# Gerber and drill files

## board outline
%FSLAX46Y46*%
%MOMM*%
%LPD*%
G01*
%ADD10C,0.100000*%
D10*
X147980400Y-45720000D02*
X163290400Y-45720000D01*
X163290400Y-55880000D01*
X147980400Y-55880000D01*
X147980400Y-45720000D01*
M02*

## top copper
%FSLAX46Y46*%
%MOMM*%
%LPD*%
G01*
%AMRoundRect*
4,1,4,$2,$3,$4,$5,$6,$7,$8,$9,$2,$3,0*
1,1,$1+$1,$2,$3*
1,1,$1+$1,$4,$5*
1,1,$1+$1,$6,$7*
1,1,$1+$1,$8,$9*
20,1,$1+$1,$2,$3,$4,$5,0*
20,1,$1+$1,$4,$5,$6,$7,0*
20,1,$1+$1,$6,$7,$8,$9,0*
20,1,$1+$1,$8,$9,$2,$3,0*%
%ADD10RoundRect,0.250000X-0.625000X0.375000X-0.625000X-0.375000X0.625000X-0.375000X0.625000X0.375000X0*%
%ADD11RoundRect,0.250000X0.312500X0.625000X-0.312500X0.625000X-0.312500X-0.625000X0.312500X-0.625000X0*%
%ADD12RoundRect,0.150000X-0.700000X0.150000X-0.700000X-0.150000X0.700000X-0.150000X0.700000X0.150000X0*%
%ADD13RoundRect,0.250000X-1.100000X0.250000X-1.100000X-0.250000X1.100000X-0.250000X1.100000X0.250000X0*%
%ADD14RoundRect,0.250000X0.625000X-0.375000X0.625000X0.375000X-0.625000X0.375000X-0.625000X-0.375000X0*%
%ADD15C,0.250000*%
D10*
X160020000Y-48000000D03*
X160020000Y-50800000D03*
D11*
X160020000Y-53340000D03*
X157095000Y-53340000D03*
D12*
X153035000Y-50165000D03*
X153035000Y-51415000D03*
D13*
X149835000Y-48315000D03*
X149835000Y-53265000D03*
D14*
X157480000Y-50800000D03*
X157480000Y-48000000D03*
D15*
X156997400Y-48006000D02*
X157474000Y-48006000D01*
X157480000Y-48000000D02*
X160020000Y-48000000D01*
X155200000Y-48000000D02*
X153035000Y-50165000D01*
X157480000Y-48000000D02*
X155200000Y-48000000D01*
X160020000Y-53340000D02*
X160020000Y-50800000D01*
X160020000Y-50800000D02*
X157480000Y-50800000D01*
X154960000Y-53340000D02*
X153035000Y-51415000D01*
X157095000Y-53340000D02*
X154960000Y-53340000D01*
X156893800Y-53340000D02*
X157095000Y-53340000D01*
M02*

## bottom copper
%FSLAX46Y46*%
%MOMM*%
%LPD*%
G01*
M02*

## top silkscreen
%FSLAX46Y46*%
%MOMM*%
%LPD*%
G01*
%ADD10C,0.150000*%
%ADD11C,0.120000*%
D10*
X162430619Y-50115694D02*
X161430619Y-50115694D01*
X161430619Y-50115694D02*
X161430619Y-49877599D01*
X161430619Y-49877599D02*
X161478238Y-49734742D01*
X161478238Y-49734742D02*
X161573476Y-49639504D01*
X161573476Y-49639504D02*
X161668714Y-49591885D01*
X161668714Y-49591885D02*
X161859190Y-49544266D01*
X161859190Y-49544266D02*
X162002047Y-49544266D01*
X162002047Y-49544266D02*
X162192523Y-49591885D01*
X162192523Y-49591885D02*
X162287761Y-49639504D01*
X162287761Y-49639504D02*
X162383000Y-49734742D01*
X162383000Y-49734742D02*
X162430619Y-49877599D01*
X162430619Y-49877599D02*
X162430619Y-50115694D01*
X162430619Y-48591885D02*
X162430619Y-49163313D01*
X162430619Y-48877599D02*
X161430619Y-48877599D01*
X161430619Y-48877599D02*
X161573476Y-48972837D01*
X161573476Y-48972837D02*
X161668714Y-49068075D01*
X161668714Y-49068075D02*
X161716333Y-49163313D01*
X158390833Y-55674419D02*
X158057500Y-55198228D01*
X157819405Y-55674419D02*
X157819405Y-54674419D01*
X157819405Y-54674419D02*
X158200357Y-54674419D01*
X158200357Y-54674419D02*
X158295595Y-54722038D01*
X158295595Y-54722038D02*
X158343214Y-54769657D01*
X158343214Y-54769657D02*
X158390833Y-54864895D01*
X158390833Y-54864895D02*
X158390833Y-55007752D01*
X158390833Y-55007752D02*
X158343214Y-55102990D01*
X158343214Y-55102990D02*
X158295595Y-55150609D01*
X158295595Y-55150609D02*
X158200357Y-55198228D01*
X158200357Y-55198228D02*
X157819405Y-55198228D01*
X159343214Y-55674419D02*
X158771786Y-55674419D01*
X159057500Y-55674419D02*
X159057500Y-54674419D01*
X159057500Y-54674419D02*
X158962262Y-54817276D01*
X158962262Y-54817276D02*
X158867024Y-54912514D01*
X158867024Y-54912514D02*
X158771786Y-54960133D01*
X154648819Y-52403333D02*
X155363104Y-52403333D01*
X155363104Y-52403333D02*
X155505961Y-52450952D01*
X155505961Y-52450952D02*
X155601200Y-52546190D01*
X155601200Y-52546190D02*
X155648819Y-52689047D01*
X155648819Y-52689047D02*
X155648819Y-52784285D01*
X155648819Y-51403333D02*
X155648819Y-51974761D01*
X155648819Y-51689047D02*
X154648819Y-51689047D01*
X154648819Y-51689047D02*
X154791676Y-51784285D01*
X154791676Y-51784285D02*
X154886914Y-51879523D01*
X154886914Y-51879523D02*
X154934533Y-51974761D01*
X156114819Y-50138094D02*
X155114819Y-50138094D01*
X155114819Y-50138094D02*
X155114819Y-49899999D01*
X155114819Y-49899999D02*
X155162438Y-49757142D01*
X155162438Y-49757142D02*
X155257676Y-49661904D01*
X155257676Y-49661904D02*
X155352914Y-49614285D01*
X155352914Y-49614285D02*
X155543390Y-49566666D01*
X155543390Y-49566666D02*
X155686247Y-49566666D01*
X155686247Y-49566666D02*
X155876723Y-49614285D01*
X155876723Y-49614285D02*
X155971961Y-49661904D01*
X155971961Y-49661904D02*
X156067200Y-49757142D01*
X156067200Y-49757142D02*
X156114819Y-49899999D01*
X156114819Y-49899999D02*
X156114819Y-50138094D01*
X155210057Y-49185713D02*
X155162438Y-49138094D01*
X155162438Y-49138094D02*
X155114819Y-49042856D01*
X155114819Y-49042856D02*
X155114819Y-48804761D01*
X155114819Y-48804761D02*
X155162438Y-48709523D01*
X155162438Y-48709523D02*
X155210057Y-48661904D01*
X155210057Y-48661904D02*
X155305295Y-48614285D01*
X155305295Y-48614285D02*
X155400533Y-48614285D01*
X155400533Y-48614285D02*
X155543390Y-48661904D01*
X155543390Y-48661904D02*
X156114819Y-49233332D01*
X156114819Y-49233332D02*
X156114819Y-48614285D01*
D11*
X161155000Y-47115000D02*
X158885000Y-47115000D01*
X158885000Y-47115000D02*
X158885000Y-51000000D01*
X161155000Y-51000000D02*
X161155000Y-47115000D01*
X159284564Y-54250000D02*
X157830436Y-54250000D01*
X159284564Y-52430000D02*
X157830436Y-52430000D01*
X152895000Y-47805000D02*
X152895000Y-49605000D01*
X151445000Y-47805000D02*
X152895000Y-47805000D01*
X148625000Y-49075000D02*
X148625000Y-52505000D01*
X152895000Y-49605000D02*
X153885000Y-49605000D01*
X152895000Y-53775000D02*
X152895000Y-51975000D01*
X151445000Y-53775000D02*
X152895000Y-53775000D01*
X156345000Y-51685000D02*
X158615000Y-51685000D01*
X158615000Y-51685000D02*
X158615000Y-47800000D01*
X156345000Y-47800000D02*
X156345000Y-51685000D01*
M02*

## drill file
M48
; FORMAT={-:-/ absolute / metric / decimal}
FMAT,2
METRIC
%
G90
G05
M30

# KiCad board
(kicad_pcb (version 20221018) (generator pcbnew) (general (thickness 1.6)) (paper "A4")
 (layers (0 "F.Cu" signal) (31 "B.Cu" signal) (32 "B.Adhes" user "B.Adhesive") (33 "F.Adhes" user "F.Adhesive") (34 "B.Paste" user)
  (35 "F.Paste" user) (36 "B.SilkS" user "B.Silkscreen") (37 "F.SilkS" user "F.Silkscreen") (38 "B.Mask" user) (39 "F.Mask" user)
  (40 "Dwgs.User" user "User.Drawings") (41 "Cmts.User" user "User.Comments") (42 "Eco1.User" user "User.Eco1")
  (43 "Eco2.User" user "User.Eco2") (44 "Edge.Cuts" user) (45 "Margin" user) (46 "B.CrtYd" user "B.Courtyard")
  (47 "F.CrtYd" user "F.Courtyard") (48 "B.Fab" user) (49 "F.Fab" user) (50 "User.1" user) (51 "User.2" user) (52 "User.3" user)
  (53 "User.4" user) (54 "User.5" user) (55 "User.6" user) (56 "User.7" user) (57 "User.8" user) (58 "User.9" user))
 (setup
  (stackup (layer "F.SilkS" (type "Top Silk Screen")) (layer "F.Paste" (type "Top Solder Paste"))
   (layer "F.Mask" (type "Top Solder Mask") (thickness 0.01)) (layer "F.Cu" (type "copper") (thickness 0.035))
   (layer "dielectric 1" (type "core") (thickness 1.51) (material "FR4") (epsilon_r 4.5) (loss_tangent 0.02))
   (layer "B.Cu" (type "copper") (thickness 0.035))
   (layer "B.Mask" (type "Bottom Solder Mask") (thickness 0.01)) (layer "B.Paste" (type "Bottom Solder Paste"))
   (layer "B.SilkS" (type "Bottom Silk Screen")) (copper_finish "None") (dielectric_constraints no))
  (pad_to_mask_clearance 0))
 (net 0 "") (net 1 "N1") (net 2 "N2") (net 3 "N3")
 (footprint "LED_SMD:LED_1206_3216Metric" (layer "F.Cu") (at 160.02 49.4 -90)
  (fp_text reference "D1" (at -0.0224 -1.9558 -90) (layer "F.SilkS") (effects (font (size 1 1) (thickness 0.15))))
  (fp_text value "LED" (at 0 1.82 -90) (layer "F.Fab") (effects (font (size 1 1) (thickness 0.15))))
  (fp_line (start -2.285 -1.135) (end -2.285 1.135) (stroke (width 0.12) (type solid)) (layer "F.SilkS"))
  (fp_line (start -2.285 1.135) (end 1.6 1.135) (stroke (width 0.12) (type solid)) (layer "F.SilkS"))
  (fp_line (start 1.6 -1.135) (end -2.285 -1.135) (stroke (width 0.12) (type solid)) (layer "F.SilkS"))
  (pad "1" smd roundrect (at -1.4 0 270) (size 1.25 1.75) (layers "F.Cu" "F.Paste" "F.Mask") (roundrect_rratio 0.2) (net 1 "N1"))
  (pad "2" smd roundrect (at 1.4 0 270) (size 1.25 1.75) (layers "F.Cu" "F.Paste" "F.Mask") (roundrect_rratio 0.2) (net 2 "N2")))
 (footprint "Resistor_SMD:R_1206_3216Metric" (layer "F.Cu") (at 158.5575 53.34 180)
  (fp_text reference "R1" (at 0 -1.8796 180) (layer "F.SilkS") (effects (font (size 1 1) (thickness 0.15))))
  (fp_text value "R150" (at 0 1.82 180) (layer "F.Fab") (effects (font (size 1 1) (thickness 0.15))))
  (fp_line (start -0.727064 -0.91) (end 0.727064 -0.91) (stroke (width 0.12) (type solid)) (layer "F.SilkS"))
  (fp_line (start -0.727064 0.91) (end 0.727064 0.91) (stroke (width 0.12) (type solid)) (layer "F.SilkS"))
  (pad "1" smd roundrect (at -1.4625 0 180) (size 1.125 1.75) (layers "F.Cu" "F.Paste" "F.Mask") (roundrect_rratio 0.2222222222)
   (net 2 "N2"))
  (pad "2" smd roundrect (at 1.4625 0 180) (size 1.125 1.75) (layers "F.Cu" "F.Paste" "F.Mask") (roundrect_rratio 0.2222222222) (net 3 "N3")))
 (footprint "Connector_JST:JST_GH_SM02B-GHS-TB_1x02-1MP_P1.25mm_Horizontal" (layer "F.Cu") (at 151.185 50.79 -90)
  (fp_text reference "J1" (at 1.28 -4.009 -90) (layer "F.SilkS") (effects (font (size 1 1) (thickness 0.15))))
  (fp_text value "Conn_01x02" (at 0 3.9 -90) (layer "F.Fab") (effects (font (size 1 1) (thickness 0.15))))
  (fp_line (start -2.985 -1.71) (end -1.185 -1.71) (stroke (width 0.12) (type solid)) (layer "F.SilkS"))
  (fp_line (start -2.985 -0.26) (end -2.985 -1.71) (stroke (width 0.12) (type solid)) (layer "F.SilkS"))
  (fp_line (start -1.715 2.56) (end 1.715 2.56) (stroke (width 0.12) (type solid)) (layer "F.SilkS"))
  (fp_line (start -1.185 -1.71) (end -1.185 -2.7) (stroke (width 0.12) (type solid)) (layer "F.SilkS"))
  (fp_line (start 2.985 -1.71) (end 1.185 -1.71) (stroke (width 0.12) (type solid)) (layer "F.SilkS"))
  (fp_line (start 2.985 -0.26) (end 2.985 -1.71) (stroke (width 0.12) (type solid)) (layer "F.SilkS"))
  (pad "1" smd roundrect (at -0.625 -1.85 270) (size 0.6 1.7) (layers "F.Cu" "F.Paste" "F.Mask") (roundrect_rratio 0.25) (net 1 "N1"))
  (pad "2" smd roundrect (at 0.625 -1.85 270) (size 0.6 1.7) (layers "F.Cu" "F.Paste" "F.Mask") (roundrect_rratio 0.25) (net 3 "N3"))
  (pad "MP" smd roundrect (at -2.475 1.35 270) (size 1 2.7) (layers "F.Cu" "F.Paste" "F.Mask") (roundrect_rratio 0.25))
  (pad "MP" smd roundrect (at 2.475 1.35 270) (size 1 2.7) (layers "F.Cu" "F.Paste" "F.Mask") (roundrect_rratio 0.25)))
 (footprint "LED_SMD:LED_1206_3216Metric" (layer "F.Cu") (at 157.48 49.4 90)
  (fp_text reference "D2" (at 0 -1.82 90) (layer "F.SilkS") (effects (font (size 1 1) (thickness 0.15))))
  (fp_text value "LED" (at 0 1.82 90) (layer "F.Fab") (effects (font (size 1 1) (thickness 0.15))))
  (fp_line (start -2.285 -1.135) (end -2.285 1.135) (stroke (width 0.12) (type solid)) (layer "F.SilkS"))
  (fp_line (start -2.285 1.135) (end 1.6 1.135) (stroke (width 0.12) (type solid)) (layer "F.SilkS"))
  (fp_line (start 1.6 -1.135) (end -2.285 -1.135) (stroke (width 0.12) (type solid)) (layer "F.SilkS"))
  (pad "1" smd roundrect (at -1.4 0 90) (size 1.25 1.75) (layers "F.Cu" "F.Paste" "F.Mask") (roundrect_rratio 0.2) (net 2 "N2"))
  (pad "2" smd roundrect (at 1.4 0 90) (size 1.25 1.75) (layers "F.Cu" "F.Paste" "F.Mask") (roundrect_rratio 0.2) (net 1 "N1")))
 (gr_rect (start 147.9804 45.72) (end 163.2904 55.88) (stroke (width 0.1) (type default)) (fill none) (layer "Edge.Cuts"))
 (segment (start 156.9974 48.006) (end 157.474 48.006) (width 0.25) (layer "F.Cu") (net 1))
 (segment (start 157.48 48) (end 160.02 48) (width 0.25) (layer "F.Cu") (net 1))
 (segment (start 155.2 48) (end 153.035 50.165) (width 0.25) (layer "F.Cu") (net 1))
 (segment (start 157.48 48) (end 155.2 48) (width 0.25) (layer "F.Cu") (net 1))
 (segment (start 160.02 53.34) (end 160.02 50.8) (width 0.25) (layer "F.Cu") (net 2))
 (segment (start 160.02 50.8) (end 157.48 50.8) (width 0.25) (layer "F.Cu") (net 2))
 (segment (start 154.96 53.34) (end 153.035 51.415) (width 0.25) (layer "F.Cu") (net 3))
 (segment (start 157.095 53.34) (end 154.96 53.34) (width 0.25) (layer "F.Cu") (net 3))
 (segment (start 156.8938 53.34) (end 157.095 53.34) (width 0.25) (layer "F.Cu") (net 3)))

